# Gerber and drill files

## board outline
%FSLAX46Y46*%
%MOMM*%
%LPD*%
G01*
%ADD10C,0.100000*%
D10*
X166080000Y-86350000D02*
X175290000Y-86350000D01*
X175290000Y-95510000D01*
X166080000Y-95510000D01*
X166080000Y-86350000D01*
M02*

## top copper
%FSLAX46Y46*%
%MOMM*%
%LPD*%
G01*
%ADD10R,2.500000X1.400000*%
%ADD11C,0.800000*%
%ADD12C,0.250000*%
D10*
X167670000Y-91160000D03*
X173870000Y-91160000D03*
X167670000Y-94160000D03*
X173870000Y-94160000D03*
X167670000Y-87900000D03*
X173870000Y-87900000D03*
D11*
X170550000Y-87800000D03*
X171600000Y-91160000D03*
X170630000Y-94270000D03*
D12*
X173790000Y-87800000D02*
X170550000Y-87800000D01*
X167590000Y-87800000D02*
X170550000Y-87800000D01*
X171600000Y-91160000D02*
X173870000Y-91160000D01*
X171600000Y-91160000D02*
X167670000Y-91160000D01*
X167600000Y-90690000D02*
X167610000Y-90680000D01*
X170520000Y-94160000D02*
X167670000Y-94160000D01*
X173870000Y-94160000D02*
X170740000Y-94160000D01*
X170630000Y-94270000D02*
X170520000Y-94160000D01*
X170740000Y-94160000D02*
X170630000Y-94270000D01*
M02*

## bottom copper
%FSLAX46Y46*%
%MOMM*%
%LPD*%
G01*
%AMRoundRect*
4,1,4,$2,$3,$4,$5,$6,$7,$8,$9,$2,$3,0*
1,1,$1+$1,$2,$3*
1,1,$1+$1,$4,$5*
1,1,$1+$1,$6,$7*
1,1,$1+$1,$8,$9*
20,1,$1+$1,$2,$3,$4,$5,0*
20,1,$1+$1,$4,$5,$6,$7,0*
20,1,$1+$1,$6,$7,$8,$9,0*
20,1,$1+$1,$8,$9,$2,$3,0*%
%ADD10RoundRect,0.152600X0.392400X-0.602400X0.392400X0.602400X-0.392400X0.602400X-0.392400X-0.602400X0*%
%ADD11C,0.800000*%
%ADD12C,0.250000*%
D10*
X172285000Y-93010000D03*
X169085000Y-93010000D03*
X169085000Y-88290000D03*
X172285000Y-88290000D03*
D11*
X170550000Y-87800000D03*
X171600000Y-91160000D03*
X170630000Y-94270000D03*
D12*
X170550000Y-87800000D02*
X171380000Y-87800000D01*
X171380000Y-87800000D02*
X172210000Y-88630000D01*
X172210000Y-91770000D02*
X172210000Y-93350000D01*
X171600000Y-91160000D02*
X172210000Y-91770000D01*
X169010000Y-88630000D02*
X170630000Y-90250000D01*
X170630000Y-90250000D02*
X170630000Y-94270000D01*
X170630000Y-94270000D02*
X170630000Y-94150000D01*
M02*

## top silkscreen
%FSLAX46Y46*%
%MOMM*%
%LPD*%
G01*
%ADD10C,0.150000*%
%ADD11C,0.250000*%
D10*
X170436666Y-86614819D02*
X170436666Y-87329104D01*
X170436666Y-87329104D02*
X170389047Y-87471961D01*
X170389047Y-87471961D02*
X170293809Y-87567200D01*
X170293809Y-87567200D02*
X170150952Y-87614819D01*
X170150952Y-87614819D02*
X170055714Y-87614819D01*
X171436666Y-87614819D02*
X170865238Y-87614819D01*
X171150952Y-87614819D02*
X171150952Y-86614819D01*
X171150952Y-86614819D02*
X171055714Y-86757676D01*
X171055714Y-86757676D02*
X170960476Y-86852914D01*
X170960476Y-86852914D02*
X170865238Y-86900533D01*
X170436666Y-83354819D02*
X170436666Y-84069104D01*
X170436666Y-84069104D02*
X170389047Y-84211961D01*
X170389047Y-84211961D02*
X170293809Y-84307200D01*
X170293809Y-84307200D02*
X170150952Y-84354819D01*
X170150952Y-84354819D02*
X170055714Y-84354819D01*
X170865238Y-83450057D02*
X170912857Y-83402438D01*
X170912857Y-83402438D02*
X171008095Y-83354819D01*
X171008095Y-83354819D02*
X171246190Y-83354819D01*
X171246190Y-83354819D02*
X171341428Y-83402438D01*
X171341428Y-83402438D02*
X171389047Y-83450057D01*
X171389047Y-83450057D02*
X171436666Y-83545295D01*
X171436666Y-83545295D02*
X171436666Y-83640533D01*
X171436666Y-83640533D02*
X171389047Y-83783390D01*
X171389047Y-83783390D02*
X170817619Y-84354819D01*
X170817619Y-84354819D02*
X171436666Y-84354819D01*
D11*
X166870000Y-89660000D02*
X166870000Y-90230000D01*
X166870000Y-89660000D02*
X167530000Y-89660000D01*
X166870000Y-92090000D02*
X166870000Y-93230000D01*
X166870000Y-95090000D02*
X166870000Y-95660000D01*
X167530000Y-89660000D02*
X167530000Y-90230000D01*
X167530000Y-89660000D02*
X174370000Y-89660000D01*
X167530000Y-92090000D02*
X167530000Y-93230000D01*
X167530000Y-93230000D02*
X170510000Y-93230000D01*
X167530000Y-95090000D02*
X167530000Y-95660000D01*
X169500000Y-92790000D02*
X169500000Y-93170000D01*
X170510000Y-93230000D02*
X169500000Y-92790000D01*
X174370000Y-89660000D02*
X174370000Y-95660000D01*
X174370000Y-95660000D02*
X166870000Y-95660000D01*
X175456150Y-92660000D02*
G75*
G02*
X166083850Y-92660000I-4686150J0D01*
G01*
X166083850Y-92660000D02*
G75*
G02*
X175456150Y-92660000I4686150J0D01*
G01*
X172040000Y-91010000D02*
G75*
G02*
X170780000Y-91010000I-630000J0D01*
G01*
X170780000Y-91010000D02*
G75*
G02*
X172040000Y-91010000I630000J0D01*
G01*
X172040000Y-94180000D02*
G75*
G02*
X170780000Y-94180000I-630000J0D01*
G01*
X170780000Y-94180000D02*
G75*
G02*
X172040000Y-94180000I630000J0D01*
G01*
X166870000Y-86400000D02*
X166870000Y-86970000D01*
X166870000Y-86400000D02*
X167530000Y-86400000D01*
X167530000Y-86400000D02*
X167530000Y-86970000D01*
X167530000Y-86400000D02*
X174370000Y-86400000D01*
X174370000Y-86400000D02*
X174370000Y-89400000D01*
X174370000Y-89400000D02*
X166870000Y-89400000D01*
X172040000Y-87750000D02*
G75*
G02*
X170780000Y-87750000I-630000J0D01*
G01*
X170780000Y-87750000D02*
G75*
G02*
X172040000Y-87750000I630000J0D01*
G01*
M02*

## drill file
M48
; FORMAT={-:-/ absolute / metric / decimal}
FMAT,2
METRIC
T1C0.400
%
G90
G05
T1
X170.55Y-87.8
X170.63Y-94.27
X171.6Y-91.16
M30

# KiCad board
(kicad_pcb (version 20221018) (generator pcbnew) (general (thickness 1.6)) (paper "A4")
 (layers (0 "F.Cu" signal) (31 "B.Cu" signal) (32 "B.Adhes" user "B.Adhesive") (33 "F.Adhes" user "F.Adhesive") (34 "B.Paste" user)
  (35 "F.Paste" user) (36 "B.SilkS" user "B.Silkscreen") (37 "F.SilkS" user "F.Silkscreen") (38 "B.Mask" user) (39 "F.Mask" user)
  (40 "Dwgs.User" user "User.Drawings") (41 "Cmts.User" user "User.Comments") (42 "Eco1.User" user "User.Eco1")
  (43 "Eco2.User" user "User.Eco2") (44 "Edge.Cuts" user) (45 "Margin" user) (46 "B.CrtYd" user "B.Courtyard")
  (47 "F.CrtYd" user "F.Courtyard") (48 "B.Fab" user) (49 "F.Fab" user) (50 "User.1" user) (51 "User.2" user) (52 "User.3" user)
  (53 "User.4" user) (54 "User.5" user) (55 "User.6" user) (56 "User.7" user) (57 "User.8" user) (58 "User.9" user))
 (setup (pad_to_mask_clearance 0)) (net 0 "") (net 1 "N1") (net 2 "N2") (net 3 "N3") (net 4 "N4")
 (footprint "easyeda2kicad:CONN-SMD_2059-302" (layer "F.Cu") (at 170.77 92.66)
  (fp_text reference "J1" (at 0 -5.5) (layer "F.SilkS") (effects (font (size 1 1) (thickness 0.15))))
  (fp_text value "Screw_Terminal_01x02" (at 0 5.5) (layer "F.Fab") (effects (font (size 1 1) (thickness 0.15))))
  (fp_line (start -3.9 -3) (end -3.9 -2.43) (stroke (width 0.25) (type solid)) (layer "F.SilkS"))
  (fp_line (start -3.9 -3) (end -3.24 -3) (stroke (width 0.25) (type solid)) (layer "F.SilkS"))
  (fp_line (start -3.9 -0.57) (end -3.9 0.57) (stroke (width 0.25) (type solid)) (layer "F.SilkS"))
  (fp_line (start -3.9 2.43) (end -3.9 3) (stroke (width 0.25) (type solid)) (layer "F.SilkS"))
  (fp_line (start -3.24 -3) (end -3.24 -2.43) (stroke (width 0.25) (type solid)) (layer "F.SilkS"))
  (fp_line (start -3.24 -3) (end 3.6 -3) (stroke (width 0.25) (type solid)) (layer "F.SilkS"))
  (fp_line (start -3.24 -0.57) (end -3.24 0.57) (stroke (width 0.25) (type solid)) (layer "F.SilkS"))
  (fp_line (start -3.24 0.57) (end -0.26 0.57) (stroke (width 0.25) (type solid)) (layer "F.SilkS"))
  (fp_line (start -3.24 2.43) (end -3.24 3) (stroke (width 0.25) (type solid)) (layer "F.SilkS"))
  (fp_line (start -1.27 0.13) (end -1.27 0.51) (stroke (width 0.25) (type solid)) (layer "F.SilkS"))
  (fp_line (start -0.26 0.57) (end -1.27 0.13) (stroke (width 0.25) (type solid)) (layer "F.SilkS"))
  (fp_line (start 3.6 -3) (end 3.6 3) (stroke (width 0.25) (type solid)) (layer "F.SilkS"))
  (fp_line (start 3.6 3) (end -3.9 3) (stroke (width 0.25) (type solid)) (layer "F.SilkS"))
  (fp_arc (start 3.6 -3) (mid -3.6 3) (end 3.6 -3) (stroke (width 0.25) (type solid)) (layer "F.SilkS"))
  (fp_circle (center 0.64 -1.65) (end 1.27 -1.65) (stroke (width 0.25) (type solid)) (fill none) (layer "F.SilkS"))
  (fp_circle (center 0.64 1.52) (end 1.27 1.52) (stroke (width 0.25) (type solid)) (fill none) (layer "F.SilkS"))
  (pad "1" smd rect (at -3.1 -1.5 90) (size 1.4 2.5) (layers "F.Cu" "F.Paste" "F.Mask") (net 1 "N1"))
  (pad "1" smd rect (at 3.1 -1.5 90) (size 1.4 2.5) (layers "F.Cu" "F.Paste" "F.Mask") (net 1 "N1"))
  (pad "2" smd rect (at -3.1 1.5 90) (size 1.4 2.5) (layers "F.Cu" "F.Paste" "F.Mask") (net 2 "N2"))
  (pad "2" smd rect (at 3.1 1.5 90) (size 1.4 2.5) (layers "F.Cu" "F.Paste" "F.Mask") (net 2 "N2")))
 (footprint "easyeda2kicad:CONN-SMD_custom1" (layer "F.Cu") (at 170.77 89.4)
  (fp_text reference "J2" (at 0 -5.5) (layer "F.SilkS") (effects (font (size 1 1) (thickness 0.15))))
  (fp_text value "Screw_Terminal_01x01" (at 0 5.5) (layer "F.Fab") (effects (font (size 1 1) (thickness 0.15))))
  (fp_line (start -3.9 -3) (end -3.9 -2.43) (stroke (width 0.25) (type solid)) (layer "F.SilkS"))
  (fp_line (start -3.9 -3) (end -3.24 -3) (stroke (width 0.25) (type solid)) (layer "F.SilkS"))
  (fp_line (start -3.24 -3) (end -3.24 -2.43) (stroke (width 0.25) (type solid)) (layer "F.SilkS"))
  (fp_line (start -3.24 -3) (end 3.6 -3) (stroke (width 0.25) (type solid)) (layer "F.SilkS"))
  (fp_line (start 3.6 -3) (end 3.6 0) (stroke (width 0.25) (type solid)) (layer "F.SilkS"))
  (fp_line (start 3.6 0) (end -3.9 0) (stroke (width 0.25) (type solid)) (layer "F.SilkS"))
  (fp_circle (center 0.64 -1.65) (end 1.27 -1.65) (stroke (width 0.25) (type solid)) (fill none) (layer "F.SilkS"))
  (pad "1" smd rect (at -3.1 -1.5 90) (size 1.4 2.5) (layers "F.Cu" "F.Paste" "F.Mask") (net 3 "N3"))
  (pad "1" smd rect (at 3.1 -1.5 90) (size 1.4 2.5) (layers "F.Cu" "F.Paste" "F.Mask") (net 3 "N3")))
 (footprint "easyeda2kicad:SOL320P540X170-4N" (layer "B.Cu") (at 170.685 90.65 90)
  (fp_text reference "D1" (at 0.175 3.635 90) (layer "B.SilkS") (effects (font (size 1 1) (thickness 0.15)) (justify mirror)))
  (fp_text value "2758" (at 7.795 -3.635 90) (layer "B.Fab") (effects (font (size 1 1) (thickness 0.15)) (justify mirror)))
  (pad "1" smd roundrect (at -2.36 1.6 90) (size 1.51 1.09) (layers "B.Cu" "B.Paste" "B.Mask") (roundrect_rratio 0.14) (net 1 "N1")
   (solder_mask_margin 0.102))
  (pad "2" smd roundrect (at -2.36 -1.6 90) (size 1.51 1.09) (layers "B.Cu" "B.Paste" "B.Mask") (roundrect_rratio 0.14) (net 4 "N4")
   (solder_mask_margin 0.102))
  (pad "3" smd roundrect (at 2.36 -1.6 90) (size 1.51 1.09) (layers "B.Cu" "B.Paste" "B.Mask") (roundrect_rratio 0.14) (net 2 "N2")
   (solder_mask_margin 0.102))
  (pad "4" smd roundrect (at 2.36 1.6 90) (size 1.51 1.09) (layers "B.Cu" "B.Paste" "B.Mask") (roundrect_rratio 0.14) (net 3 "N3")
   (solder_mask_margin 0.102)))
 (gr_rect (start 166.08 86.35) (end 175.29 95.51) (stroke (width 0.1) (type default)) (fill none) (layer "Edge.Cuts"))
 (segment (start 173.79 87.8) (end 170.55 87.8) (width 0.25) (layer "F.Cu") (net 3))
 (segment (start 167.59 87.8) (end 170.55 87.8) (width 0.25) (layer "F.Cu") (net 3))
 (via (at 170.55 87.8) (size 0.8) (drill 0.4) (layers "F.Cu" "B.Cu") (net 3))
 (segment (start 170.55 87.8) (end 171.38 87.8) (width 0.25) (layer "B.Cu") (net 3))
 (segment (start 171.38 87.8) (end 172.21 88.63) (width 0.25) (layer "B.Cu") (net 3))
 (segment (start 171.6 91.16) (end 173.87 91.16) (width 0.25) (layer "F.Cu") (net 1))
 (segment (start 171.6 91.16) (end 167.67 91.16) (width 0.25) (layer "F.Cu") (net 1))
 (segment (start 167.6 90.69) (end 167.61 90.68) (width 0.25) (layer "F.Cu") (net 1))
 (via (at 171.6 91.16) (size 0.8) (drill 0.4) (layers "F.Cu" "B.Cu") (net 1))
 (segment (start 172.21 91.77) (end 172.21 93.35) (width 0.25) (layer "B.Cu") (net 1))
 (segment (start 171.6 91.16) (end 172.21 91.77) (width 0.25) (layer "B.Cu") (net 1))
 (segment (start 170.52 94.16) (end 167.67 94.16) (width 0.25) (layer "F.Cu") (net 2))
 (segment (start 173.87 94.16) (end 170.74 94.16) (width 0.25) (layer "F.Cu") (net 2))
 (segment (start 170.63 94.27) (end 170.52 94.16) (width 0.25) (layer "F.Cu") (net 2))
 (segment (start 170.74 94.16) (end 170.63 94.27) (width 0.25) (layer "F.Cu") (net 2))
 (via (at 170.63 94.27) (size 0.8) (drill 0.4) (layers "F.Cu" "B.Cu") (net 2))
 (segment (start 169.01 88.63) (end 170.63 90.25) (width 0.25) (layer "B.Cu") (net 2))
 (segment (start 170.63 90.25) (end 170.63 94.27) (width 0.25) (layer "B.Cu") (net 2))
 (segment (start 170.63 94.27) (end 170.63 94.15) (width 0.25) (layer "B.Cu") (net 2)))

